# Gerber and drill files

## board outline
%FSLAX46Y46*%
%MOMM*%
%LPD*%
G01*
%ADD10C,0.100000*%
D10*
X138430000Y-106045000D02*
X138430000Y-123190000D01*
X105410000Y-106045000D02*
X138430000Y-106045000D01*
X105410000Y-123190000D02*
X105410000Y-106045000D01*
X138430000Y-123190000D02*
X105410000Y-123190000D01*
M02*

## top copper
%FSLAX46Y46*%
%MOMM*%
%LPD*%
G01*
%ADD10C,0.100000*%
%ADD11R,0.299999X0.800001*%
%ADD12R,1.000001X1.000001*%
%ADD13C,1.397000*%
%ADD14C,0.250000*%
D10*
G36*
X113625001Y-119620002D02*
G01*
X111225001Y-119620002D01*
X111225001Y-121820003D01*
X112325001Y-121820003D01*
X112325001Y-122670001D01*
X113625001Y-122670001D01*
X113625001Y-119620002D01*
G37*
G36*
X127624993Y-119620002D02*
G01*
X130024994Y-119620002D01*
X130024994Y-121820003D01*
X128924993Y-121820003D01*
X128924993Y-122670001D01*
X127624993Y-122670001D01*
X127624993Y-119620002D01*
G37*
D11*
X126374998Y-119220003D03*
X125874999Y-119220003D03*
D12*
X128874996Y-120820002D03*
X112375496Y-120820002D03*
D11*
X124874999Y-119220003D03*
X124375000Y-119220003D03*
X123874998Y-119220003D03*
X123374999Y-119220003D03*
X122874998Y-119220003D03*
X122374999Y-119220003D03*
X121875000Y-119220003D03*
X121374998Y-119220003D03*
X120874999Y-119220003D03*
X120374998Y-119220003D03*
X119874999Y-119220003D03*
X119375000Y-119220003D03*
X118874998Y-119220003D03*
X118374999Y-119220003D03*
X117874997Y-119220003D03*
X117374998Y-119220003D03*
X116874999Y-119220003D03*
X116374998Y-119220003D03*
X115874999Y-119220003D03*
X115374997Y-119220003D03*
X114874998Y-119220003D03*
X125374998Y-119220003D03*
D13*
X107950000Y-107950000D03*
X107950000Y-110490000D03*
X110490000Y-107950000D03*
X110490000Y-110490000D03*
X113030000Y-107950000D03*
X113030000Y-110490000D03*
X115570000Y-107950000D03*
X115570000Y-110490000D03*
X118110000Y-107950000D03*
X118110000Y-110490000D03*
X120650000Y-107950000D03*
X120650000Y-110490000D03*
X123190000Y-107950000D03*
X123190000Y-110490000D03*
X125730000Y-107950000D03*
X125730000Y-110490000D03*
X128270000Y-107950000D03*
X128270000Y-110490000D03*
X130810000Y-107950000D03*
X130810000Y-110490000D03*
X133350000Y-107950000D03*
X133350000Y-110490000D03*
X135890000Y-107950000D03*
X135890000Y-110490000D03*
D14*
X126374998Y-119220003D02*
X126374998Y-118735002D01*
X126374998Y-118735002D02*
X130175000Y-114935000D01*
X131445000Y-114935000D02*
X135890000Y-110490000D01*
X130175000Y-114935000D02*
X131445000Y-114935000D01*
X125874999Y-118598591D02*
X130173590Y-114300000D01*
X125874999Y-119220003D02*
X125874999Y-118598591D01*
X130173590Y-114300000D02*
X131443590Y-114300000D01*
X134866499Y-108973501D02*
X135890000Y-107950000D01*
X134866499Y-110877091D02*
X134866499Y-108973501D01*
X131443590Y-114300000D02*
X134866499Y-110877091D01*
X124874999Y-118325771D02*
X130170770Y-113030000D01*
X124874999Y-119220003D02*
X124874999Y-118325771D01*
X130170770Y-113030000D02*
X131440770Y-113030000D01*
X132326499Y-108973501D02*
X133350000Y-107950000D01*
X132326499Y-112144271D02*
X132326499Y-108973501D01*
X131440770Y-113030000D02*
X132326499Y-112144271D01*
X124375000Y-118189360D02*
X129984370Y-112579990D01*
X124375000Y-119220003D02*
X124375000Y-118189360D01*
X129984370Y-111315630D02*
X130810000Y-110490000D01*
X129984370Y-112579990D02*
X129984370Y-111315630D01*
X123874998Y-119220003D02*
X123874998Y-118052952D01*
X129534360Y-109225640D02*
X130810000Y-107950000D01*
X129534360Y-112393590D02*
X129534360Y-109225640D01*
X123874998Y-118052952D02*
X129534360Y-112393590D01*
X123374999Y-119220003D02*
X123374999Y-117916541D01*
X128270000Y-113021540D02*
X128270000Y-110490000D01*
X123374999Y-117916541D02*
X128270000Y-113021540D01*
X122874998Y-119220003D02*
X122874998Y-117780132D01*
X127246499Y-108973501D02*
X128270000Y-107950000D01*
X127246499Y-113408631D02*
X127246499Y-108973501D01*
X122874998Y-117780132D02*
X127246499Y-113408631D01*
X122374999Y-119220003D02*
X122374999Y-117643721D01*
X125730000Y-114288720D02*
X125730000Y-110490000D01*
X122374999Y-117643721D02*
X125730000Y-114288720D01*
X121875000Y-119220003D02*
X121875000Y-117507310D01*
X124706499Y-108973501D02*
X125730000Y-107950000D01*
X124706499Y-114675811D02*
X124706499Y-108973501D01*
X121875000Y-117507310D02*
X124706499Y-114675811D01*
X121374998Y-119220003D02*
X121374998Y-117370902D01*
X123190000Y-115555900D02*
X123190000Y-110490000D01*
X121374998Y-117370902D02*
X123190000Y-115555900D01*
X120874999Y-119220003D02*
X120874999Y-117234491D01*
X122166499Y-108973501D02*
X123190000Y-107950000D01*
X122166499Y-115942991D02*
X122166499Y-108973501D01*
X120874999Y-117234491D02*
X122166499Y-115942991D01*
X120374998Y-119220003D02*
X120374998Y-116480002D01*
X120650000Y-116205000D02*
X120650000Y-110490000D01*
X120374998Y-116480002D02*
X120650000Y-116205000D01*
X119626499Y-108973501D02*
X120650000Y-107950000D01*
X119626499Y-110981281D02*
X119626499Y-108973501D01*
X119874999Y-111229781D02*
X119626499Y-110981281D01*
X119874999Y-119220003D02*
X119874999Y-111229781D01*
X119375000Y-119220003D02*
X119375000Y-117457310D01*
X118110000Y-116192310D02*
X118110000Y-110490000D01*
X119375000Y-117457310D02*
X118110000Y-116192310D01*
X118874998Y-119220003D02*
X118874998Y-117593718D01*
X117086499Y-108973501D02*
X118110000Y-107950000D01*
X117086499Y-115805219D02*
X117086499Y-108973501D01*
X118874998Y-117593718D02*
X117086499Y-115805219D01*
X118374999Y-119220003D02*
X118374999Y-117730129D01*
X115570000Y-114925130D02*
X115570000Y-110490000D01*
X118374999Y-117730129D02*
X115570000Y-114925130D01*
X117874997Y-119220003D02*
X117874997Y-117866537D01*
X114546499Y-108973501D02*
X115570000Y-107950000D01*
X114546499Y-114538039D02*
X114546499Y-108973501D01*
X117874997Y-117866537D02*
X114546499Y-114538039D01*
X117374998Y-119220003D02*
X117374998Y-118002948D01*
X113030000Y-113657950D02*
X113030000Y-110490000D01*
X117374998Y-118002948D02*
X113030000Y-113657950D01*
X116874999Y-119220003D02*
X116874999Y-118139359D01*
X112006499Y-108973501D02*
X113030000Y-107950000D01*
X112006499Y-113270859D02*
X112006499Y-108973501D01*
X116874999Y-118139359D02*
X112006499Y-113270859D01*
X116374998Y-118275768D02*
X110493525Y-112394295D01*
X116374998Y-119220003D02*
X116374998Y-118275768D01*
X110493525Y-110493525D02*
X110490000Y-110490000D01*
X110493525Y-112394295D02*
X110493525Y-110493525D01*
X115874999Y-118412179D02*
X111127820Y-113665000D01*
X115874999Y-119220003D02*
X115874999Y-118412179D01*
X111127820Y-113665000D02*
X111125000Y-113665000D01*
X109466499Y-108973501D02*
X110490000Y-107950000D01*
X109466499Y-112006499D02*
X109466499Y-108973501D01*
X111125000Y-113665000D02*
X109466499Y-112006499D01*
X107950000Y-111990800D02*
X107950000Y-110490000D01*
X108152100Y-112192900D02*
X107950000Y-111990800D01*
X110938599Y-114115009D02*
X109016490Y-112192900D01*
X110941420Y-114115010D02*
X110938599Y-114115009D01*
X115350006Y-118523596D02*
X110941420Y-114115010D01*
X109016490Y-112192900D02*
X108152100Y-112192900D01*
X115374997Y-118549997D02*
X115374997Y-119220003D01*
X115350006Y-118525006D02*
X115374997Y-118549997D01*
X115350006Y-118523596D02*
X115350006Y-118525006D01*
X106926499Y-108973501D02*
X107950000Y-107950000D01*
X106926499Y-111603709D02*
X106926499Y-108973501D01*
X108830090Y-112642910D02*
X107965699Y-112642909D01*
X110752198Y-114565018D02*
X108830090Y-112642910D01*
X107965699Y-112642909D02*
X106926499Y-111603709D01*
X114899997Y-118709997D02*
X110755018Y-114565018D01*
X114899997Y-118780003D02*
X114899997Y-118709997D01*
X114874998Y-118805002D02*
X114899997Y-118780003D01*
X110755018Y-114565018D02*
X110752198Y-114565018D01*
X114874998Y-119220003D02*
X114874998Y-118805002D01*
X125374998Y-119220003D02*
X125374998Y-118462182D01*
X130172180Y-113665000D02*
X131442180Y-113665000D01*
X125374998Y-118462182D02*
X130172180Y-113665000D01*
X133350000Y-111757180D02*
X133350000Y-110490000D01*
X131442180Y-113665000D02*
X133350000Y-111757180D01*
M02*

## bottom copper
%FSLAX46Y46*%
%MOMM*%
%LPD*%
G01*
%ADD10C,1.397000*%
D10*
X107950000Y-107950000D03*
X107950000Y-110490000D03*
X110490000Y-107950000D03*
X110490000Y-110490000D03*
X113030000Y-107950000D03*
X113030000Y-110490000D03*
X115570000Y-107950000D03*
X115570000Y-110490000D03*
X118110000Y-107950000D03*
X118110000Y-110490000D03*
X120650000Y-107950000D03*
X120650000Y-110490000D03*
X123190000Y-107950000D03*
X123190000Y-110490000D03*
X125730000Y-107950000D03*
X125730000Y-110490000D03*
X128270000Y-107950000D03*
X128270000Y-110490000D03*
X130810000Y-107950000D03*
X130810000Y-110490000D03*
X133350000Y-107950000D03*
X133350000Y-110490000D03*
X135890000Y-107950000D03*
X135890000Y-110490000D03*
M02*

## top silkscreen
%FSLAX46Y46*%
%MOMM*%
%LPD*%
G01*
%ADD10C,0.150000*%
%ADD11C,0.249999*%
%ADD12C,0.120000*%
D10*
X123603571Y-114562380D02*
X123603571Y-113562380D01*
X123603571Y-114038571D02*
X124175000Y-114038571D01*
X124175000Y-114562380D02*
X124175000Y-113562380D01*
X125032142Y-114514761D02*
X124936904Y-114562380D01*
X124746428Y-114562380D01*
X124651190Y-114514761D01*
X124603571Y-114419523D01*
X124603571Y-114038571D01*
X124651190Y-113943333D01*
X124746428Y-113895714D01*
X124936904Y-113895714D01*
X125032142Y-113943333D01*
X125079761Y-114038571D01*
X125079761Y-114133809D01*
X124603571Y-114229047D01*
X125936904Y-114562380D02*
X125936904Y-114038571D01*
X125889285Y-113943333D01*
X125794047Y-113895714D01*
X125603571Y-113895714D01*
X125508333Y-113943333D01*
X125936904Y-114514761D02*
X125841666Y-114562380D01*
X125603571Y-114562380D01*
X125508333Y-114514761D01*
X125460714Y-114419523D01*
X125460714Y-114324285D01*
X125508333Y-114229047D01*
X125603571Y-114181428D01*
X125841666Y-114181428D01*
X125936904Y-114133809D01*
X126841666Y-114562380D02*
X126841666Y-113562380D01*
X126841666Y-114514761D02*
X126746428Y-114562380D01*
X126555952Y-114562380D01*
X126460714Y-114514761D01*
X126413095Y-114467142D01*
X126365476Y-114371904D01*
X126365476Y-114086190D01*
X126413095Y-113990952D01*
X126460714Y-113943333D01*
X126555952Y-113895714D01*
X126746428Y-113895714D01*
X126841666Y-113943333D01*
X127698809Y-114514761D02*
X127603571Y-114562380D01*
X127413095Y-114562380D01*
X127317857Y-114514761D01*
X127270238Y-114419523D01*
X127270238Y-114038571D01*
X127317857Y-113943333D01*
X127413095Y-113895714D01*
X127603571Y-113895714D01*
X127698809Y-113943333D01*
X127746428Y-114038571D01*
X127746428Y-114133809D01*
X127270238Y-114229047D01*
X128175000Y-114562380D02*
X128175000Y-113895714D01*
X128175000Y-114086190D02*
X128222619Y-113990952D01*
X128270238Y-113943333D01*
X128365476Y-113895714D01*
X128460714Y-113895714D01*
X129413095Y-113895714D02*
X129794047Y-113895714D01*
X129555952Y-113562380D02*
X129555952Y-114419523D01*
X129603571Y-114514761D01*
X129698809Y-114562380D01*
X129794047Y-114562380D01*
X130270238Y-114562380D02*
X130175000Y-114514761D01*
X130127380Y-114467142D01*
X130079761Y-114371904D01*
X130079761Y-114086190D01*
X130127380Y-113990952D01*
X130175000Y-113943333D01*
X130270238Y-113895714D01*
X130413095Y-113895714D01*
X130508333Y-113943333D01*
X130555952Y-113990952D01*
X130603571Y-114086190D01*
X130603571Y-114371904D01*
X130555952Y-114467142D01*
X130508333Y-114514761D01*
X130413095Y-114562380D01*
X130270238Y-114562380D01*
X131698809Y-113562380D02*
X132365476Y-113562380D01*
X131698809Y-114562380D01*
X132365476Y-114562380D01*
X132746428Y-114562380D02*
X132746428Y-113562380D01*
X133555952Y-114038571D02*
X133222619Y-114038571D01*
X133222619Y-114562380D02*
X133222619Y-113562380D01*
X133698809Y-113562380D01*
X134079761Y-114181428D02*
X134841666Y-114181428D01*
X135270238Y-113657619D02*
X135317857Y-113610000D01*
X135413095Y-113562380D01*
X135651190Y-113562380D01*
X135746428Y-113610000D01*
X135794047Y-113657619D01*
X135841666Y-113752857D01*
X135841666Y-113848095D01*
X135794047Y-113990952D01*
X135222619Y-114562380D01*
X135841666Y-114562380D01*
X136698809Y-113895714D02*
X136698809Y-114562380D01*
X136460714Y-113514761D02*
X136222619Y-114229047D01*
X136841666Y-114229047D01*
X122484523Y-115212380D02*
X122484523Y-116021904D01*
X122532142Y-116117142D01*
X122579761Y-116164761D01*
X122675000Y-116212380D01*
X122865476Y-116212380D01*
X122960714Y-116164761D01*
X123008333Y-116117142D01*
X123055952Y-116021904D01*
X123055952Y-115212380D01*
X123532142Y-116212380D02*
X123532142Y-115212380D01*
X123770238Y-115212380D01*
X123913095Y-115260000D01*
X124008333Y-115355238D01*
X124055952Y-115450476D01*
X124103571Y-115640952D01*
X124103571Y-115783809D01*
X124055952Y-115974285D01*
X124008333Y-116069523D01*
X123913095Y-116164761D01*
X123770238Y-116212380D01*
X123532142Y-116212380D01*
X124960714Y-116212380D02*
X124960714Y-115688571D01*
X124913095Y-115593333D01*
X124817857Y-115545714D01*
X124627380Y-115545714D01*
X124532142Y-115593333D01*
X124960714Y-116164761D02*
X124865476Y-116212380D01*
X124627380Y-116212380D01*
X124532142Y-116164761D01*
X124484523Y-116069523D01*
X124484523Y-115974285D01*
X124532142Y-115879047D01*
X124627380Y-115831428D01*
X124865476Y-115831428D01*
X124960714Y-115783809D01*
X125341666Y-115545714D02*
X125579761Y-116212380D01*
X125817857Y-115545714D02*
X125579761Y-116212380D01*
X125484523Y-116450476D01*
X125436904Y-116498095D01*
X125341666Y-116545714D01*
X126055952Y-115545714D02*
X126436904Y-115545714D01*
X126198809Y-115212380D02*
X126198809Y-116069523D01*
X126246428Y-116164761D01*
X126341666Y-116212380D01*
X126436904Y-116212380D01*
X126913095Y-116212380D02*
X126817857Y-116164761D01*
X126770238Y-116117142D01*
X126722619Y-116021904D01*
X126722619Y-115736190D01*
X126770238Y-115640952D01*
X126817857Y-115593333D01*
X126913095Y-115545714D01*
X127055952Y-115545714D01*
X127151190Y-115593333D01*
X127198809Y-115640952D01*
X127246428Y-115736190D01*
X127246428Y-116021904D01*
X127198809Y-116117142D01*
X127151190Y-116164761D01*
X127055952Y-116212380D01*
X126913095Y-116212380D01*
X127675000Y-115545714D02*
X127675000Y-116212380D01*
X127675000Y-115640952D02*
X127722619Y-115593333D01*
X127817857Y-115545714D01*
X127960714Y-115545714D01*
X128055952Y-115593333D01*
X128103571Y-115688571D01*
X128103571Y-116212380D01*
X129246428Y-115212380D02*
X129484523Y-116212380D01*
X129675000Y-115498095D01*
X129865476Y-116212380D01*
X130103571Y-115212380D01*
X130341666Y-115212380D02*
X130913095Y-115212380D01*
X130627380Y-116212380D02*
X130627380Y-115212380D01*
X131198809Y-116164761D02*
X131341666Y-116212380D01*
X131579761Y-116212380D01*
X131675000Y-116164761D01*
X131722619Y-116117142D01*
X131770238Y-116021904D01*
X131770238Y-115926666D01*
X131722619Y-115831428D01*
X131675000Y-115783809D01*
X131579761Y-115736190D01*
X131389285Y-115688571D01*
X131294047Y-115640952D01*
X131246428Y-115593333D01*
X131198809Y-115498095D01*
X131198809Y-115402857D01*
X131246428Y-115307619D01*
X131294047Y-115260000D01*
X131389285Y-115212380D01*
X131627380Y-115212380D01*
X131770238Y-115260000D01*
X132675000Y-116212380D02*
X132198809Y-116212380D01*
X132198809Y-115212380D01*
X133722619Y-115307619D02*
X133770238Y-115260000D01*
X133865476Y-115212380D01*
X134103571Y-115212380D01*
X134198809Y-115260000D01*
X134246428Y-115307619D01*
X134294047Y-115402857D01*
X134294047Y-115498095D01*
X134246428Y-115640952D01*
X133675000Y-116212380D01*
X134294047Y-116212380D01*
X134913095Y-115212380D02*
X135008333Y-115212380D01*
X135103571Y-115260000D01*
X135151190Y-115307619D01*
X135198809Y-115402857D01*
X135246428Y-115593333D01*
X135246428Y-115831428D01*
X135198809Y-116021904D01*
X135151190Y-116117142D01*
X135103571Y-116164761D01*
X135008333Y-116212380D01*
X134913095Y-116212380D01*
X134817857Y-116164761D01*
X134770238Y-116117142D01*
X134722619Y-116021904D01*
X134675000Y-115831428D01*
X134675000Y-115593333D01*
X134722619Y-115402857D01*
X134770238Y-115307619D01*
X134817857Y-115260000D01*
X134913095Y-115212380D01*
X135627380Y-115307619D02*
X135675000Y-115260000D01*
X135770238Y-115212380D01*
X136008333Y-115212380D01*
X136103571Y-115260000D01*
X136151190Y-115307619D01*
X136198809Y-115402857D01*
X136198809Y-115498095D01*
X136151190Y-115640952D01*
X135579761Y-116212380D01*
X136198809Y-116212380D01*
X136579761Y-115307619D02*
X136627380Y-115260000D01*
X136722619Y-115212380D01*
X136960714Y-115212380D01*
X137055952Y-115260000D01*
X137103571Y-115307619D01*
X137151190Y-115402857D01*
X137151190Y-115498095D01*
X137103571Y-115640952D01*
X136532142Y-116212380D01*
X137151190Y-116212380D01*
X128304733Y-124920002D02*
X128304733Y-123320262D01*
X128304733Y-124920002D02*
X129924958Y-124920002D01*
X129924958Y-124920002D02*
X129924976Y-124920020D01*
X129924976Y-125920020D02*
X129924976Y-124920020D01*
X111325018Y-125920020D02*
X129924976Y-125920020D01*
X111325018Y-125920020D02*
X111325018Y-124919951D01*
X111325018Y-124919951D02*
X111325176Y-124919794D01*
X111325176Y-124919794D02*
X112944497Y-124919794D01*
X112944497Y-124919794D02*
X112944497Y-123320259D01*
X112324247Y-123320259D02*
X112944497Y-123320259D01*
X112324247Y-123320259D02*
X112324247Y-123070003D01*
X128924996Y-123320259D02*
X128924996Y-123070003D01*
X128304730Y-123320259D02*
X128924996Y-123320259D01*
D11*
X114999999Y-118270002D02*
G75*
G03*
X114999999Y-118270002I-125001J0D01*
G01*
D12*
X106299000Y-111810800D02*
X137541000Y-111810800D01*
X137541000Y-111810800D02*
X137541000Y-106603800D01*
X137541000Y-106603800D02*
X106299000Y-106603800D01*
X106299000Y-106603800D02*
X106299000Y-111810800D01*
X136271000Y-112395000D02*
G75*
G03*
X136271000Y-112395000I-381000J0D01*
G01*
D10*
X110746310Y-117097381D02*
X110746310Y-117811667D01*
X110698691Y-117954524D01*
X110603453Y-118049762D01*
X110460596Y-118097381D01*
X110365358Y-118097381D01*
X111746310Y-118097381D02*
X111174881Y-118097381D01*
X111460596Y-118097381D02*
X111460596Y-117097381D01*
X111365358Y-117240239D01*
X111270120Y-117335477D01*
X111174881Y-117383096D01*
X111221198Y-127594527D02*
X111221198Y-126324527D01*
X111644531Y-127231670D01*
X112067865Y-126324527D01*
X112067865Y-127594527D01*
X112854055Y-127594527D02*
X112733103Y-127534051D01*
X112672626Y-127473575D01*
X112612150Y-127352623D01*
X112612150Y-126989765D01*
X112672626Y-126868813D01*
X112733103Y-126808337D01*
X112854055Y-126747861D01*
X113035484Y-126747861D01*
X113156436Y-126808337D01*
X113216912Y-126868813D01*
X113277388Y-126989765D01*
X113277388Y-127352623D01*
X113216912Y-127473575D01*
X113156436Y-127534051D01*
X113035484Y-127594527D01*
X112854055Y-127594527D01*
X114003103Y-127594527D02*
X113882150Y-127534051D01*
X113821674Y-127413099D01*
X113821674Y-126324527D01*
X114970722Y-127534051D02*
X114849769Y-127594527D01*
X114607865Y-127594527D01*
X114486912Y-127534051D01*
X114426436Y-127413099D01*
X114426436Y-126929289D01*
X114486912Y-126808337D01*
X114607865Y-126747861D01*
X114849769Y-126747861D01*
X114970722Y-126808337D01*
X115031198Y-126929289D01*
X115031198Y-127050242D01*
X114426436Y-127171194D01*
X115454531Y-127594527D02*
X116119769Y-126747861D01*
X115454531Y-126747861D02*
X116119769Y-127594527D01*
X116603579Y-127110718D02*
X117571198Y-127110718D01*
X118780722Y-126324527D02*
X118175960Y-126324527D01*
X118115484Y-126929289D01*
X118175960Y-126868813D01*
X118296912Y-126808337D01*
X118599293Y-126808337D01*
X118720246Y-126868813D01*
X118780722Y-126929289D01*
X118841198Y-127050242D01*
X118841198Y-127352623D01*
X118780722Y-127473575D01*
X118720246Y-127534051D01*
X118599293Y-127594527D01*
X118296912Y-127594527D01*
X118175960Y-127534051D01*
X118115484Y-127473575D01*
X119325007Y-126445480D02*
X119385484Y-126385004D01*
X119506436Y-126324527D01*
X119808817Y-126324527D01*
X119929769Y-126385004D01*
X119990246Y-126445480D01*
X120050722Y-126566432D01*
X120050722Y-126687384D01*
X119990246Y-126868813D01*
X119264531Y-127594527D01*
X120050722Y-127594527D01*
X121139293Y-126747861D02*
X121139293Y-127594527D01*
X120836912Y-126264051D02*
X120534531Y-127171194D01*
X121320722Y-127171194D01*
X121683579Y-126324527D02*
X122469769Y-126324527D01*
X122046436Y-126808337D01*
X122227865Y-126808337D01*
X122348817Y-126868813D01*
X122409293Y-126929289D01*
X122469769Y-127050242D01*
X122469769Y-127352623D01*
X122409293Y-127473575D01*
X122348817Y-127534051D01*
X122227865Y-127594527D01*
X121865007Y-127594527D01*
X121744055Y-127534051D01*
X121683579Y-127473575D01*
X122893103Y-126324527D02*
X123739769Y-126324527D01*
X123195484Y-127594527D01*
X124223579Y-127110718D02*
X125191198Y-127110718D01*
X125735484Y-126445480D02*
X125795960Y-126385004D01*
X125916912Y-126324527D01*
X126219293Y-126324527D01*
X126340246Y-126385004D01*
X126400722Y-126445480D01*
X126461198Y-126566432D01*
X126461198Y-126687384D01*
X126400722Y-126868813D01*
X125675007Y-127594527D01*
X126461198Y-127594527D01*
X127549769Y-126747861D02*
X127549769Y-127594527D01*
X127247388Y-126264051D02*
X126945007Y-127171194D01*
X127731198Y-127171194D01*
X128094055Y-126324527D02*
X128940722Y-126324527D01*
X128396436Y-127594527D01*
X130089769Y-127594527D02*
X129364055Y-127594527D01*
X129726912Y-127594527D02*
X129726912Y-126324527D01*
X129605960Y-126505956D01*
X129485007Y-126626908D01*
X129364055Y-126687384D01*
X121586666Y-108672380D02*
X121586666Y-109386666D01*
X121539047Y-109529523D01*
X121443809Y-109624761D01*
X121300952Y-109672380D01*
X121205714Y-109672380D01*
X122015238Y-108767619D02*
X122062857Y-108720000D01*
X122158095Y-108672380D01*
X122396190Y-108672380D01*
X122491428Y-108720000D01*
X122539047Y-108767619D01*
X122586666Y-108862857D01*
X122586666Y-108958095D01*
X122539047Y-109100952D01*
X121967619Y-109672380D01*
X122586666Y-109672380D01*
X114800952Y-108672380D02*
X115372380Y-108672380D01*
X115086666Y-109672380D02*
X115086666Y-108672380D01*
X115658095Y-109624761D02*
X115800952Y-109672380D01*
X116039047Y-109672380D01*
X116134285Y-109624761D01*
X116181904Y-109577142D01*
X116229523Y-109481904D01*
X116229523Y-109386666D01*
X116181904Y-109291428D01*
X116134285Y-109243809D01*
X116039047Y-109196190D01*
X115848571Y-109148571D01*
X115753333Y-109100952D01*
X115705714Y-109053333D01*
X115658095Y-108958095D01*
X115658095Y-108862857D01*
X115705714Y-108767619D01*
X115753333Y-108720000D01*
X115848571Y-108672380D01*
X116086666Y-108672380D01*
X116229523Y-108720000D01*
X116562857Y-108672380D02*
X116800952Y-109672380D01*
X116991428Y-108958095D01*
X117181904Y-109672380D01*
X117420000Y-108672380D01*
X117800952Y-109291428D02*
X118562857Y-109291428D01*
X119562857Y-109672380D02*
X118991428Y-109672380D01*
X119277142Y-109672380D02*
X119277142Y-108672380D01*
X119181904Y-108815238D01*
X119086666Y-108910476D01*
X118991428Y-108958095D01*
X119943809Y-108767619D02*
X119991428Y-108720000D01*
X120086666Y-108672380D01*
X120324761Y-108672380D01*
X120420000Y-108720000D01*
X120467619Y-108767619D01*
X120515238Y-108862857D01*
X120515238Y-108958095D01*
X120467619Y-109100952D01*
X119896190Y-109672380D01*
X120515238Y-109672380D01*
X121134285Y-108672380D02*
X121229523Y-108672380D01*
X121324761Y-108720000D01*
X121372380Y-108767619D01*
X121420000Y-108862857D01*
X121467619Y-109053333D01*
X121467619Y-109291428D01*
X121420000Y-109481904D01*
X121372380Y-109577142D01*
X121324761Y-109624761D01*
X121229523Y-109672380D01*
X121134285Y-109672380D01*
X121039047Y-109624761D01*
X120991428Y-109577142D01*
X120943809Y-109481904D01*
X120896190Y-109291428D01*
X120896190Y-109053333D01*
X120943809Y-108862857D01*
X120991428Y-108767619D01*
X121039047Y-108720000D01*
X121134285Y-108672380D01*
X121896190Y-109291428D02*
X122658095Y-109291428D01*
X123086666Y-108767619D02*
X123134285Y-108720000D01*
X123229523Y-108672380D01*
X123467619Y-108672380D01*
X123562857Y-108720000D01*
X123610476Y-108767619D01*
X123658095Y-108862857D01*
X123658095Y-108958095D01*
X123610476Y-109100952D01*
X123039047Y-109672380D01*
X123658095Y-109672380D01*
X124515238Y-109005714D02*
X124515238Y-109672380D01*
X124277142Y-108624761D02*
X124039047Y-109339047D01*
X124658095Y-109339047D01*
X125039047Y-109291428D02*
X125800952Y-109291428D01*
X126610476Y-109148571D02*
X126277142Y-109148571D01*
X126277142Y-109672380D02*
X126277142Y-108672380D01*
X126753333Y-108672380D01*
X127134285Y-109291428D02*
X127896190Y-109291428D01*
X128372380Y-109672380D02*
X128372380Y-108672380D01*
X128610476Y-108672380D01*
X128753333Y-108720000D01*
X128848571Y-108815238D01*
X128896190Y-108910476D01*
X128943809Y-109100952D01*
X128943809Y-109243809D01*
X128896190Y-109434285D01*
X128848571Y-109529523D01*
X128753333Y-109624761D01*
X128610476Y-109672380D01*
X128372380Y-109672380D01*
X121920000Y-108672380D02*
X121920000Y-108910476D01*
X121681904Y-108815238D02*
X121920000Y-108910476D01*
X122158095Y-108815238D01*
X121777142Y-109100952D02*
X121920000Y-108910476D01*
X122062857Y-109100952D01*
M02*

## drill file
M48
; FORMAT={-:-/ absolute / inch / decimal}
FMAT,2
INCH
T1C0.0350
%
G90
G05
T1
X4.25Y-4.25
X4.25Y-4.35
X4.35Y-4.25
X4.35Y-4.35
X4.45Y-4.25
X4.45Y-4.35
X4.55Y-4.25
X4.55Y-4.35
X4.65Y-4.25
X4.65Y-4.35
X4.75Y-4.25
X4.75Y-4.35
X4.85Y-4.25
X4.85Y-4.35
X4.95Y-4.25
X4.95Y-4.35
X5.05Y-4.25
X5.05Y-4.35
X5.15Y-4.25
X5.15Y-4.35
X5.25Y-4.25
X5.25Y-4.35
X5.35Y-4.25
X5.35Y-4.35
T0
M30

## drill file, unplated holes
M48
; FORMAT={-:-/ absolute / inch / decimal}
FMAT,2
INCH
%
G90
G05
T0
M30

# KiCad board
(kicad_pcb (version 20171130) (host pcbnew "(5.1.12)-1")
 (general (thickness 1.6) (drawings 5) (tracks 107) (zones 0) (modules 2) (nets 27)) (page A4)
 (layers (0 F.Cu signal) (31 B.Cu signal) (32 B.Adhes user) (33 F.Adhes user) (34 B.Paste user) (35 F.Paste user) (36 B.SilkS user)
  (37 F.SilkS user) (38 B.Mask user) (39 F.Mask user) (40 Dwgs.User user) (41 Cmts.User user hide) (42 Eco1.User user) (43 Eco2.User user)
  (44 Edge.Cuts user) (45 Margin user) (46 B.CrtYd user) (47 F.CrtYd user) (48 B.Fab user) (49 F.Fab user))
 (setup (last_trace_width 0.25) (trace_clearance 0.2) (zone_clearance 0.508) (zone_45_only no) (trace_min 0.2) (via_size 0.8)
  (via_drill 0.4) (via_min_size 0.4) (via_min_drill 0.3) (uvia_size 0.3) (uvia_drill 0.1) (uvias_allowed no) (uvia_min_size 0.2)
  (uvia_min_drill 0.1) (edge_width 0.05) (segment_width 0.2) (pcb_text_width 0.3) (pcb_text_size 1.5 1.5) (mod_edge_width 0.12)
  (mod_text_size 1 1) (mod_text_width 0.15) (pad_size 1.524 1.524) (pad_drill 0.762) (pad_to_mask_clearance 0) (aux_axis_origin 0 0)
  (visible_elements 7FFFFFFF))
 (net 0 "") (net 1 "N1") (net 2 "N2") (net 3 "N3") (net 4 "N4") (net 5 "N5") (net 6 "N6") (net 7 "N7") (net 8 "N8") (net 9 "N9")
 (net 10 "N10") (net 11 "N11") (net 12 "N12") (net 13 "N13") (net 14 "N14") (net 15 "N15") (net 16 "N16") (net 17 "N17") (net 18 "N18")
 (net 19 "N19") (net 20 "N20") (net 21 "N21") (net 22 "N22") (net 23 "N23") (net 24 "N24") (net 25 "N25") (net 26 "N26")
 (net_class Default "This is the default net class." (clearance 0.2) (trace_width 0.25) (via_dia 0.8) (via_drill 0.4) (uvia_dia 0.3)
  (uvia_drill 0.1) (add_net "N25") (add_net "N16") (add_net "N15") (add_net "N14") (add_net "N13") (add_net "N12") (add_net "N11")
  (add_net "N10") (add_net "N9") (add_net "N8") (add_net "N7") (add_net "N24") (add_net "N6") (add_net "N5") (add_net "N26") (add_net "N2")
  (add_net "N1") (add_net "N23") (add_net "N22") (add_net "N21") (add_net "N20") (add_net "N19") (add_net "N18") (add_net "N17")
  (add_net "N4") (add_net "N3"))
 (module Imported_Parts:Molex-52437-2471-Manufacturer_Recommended (layer F.Cu) (at 120.625246 120.020004)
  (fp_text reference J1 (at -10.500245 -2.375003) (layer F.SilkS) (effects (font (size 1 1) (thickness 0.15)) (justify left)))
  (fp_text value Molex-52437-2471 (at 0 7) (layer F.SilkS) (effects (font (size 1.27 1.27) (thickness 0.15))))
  (fp_poly
   (pts (xy -7.000245 -0.400002) (xy -9.400245 -0.400002) (xy -9.400245 1.799999) (xy -8.300245 1.799999) (xy -8.300245 2.649997)
    (xy -7.000245 2.649997))
   (layer F.Cu) (width 0))
  (fp_poly
   (pts (xy 6.999747 -0.400002) (xy 9.399748 -0.400002) (xy 9.399748 1.799999) (xy 8.299747 1.799999) (xy 8.299747 2.649997)
    (xy 6.999747 2.649997))
   (layer F.Cu) (width 0))
  (fp_line (start 7.679487 4.899998) (end 7.679487 3.300258) (layer F.SilkS) (width 0.15))
  (fp_line (start 7.679487 4.899998) (end 9.299712 4.899998) (layer F.SilkS) (width 0.15))
  (fp_line (start 9.299712 4.899998) (end 9.29973 4.900016) (layer F.SilkS) (width 0.15))
  (fp_line (start 9.29973 5.900016) (end 9.29973 4.900016) (layer F.SilkS) (width 0.15))
  (fp_line (start -9.300228 5.900016) (end 9.29973 5.900016) (layer F.SilkS) (width 0.15))
  (fp_line (start -9.300228 5.900016) (end -9.300228 4.899947) (layer F.SilkS) (width 0.15))
  (fp_line (start -9.300228 4.899947) (end -9.30007 4.89979) (layer F.SilkS) (width 0.15))
  (fp_line (start -9.30007 4.89979) (end -7.680749 4.89979) (layer F.SilkS) (width 0.15))
  (fp_line (start -7.680749 4.89979) (end -7.680749 3.300255) (layer F.SilkS) (width 0.15))
  (fp_line (start -8.300999 3.300255) (end -7.680749 3.300255) (layer F.SilkS) (width 0.15))
  (fp_line (start -8.300999 3.300255) (end -8.300999 3.049999) (layer F.SilkS) (width 0.15))
  (fp_line (start 8.29975 3.300255) (end 8.29975 3.049999) (layer F.SilkS) (width 0.15))
  (fp_line (start 7.679484 3.300255) (end 8.29975 3.300255) (layer F.SilkS) (width 0.15))
  (fp_circle (center -5.750248 -1.750002) (end -5.625247 -1.750002) (layer F.SilkS) (width 0.249999))
  (pad 24 smd rect (at 5.749752 -0.800001) (size 0.299999 0.800001) (layers F.Cu F.Paste F.Mask) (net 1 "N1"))
  (pad 23 smd rect (at 5.249753 -0.800001) (size 0.299999 0.800001) (layers F.Cu F.Paste F.Mask) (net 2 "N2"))
  (pad MP2 smd rect (at 8.24975 0.799998 180) (size 1.000001 1.000001) (layers F.Cu F.Paste F.Mask) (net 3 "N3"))
  (pad MP1 smd rect (at -8.24975 0.799998 180) (size 1.000001 1.000001) (layers F.Cu F.Paste F.Mask) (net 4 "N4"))
  (pad 21 smd rect (at 4.249753 -0.800001 180) (size 0.299999 0.800001) (layers F.Cu F.Paste F.Mask) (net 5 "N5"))
  (pad 20 smd rect (at 3.749754 -0.800001 180) (size 0.299999 0.800001) (layers F.Cu F.Paste F.Mask) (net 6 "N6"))
  (pad 19 smd rect (at 3.249752 -0.800001 180) (size 0.299999 0.800001) (layers F.Cu F.Paste F.Mask) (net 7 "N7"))
  (pad 18 smd rect (at 2.749753 -0.800001 180) (size 0.299999 0.800001) (layers F.Cu F.Paste F.Mask) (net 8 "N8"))
  (pad 17 smd rect (at 2.249752 -0.800001 180) (size 0.299999 0.800001) (layers F.Cu F.Paste F.Mask) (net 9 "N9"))
  (pad 16 smd rect (at 1.749753 -0.800001 180) (size 0.299999 0.800001) (layers F.Cu F.Paste F.Mask) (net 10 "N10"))
  (pad 15 smd rect (at 1.249754 -0.800001 180) (size 0.299999 0.800001) (layers F.Cu F.Paste F.Mask) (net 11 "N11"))
  (pad 14 smd rect (at 0.749752 -0.800001 180) (size 0.299999 0.800001) (layers F.Cu F.Paste F.Mask) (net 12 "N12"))
  (pad 13 smd rect (at 0.249753 -0.800001 180) (size 0.299999 0.800001) (layers F.Cu F.Paste F.Mask) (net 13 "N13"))
  (pad 12 smd rect (at -0.250248 -0.800001 180) (size 0.299999 0.800001) (layers F.Cu F.Paste F.Mask) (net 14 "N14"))
  (pad 11 smd rect (at -0.750247 -0.800001 180) (size 0.299999 0.800001) (layers F.Cu F.Paste F.Mask) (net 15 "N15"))
  (pad 10 smd rect (at -1.250246 -0.800001 180) (size 0.299999 0.800001) (layers F.Cu F.Paste F.Mask) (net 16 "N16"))
  (pad 9 smd rect (at -1.750248 -0.800001 180) (size 0.299999 0.800001) (layers F.Cu F.Paste F.Mask) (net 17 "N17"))
  (pad 8 smd rect (at -2.250247 -0.800001 180) (size 0.299999 0.800001) (layers F.Cu F.Paste F.Mask) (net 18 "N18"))
  (pad 7 smd rect (at -2.750249 -0.800001 180) (size 0.299999 0.800001) (layers F.Cu F.Paste F.Mask) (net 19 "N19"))
  (pad 6 smd rect (at -3.250248 -0.800001 180) (size 0.299999 0.800001) (layers F.Cu F.Paste F.Mask) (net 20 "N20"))
  (pad 5 smd rect (at -3.750247 -0.800001 180) (size 0.299999 0.800001) (layers F.Cu F.Paste F.Mask) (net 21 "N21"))
  (pad 4 smd rect (at -4.250248 -0.800001 180) (size 0.299999 0.800001) (layers F.Cu F.Paste F.Mask) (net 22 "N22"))
  (pad 3 smd rect (at -4.750247 -0.800001 180) (size 0.299999 0.800001) (layers F.Cu F.Paste F.Mask) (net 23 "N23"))
  (pad 2 smd rect (at -5.250249 -0.800001 180) (size 0.299999 0.800001) (layers F.Cu F.Paste F.Mask) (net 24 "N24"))
  (pad 1 smd rect (at -5.750248 -0.800001 180) (size 0.299999 0.800001) (layers F.Cu F.Paste F.Mask) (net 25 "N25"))
  (pad 22 smd rect (at 4.749752 -0.800001) (size 0.299999 0.800001) (layers F.Cu F.Paste F.Mask) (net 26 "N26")))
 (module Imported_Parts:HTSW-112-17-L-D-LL (layer F.Cu) (at 121.92 109.22)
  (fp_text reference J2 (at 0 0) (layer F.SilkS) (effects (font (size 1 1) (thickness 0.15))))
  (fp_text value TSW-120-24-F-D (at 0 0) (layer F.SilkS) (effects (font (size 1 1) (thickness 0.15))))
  (fp_line (start -15.621 2.5908) (end 15.621 2.5908) (layer F.SilkS) (width 0.12))
  (fp_line (start 15.621 2.5908) (end 15.621 -2.6162) (layer F.SilkS) (width 0.12))
  (fp_line (start 15.621 -2.6162) (end -15.621 -2.6162) (layer F.SilkS) (width 0.12))
  (fp_line (start -15.621 -2.6162) (end -15.621 2.5908) (layer F.SilkS) (width 0.12))
  (fp_circle (center 13.97 3.175) (end 14.351 3.175) (layer F.SilkS) (width 0.12))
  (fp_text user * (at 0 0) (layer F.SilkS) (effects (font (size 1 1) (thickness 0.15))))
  (pad 24 thru_hole circle (at -13.97 -1.27 90) (size 1.397 1.397) (drill 0.889) (layers *.Cu *.Mask) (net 25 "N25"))
  (pad 23 thru_hole circle (at -13.97 1.27 90) (size 1.397 1.397) (drill 0.889) (layers *.Cu *.Mask) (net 24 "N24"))
  (pad 22 thru_hole circle (at -11.43 -1.27 90) (size 1.397 1.397) (drill 0.889) (layers *.Cu *.Mask) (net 23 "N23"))
  (pad 21 thru_hole circle (at -11.43 1.27 90) (size 1.397 1.397) (drill 0.889) (layers *.Cu *.Mask) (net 22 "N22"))
  (pad 20 thru_hole circle (at -8.89 -1.27 90) (size 1.397 1.397) (drill 0.889) (layers *.Cu *.Mask) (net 21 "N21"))
  (pad 19 thru_hole circle (at -8.89 1.27 90) (size 1.397 1.397) (drill 0.889) (layers *.Cu *.Mask) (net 20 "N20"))
  (pad 18 thru_hole circle (at -6.35 -1.27 90) (size 1.397 1.397) (drill 0.889) (layers *.Cu *.Mask) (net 19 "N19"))
  (pad 17 thru_hole circle (at -6.35 1.27 90) (size 1.397 1.397) (drill 0.889) (layers *.Cu *.Mask) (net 18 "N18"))
  (pad 16 thru_hole circle (at -3.81 -1.27 90) (size 1.397 1.397) (drill 0.889) (layers *.Cu *.Mask) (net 17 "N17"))
  (pad 15 thru_hole circle (at -3.81 1.27 90) (size 1.397 1.397) (drill 0.889) (layers *.Cu *.Mask) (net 16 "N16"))
  (pad 14 thru_hole circle (at -1.27 -1.27 90) (size 1.397 1.397) (drill 0.889) (layers *.Cu *.Mask) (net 15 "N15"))
  (pad 13 thru_hole circle (at -1.27 1.27 90) (size 1.397 1.397) (drill 0.889) (layers *.Cu *.Mask) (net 14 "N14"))
  (pad 12 thru_hole circle (at 1.27 -1.27 90) (size 1.397 1.397) (drill 0.889) (layers *.Cu *.Mask) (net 13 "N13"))
  (pad 11 thru_hole circle (at 1.27 1.27 90) (size 1.397 1.397) (drill 0.889) (layers *.Cu *.Mask) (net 12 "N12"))
  (pad 10 thru_hole circle (at 3.81 -1.27 90) (size 1.397 1.397) (drill 0.889) (layers *.Cu *.Mask) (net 11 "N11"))
  (pad 9 thru_hole circle (at 3.81 1.27 90) (size 1.397 1.397) (drill 0.889) (layers *.Cu *.Mask) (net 10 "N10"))
  (pad 8 thru_hole circle (at 6.35 -1.27 90) (size 1.397 1.397) (drill 0.889) (layers *.Cu *.Mask) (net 9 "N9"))
  (pad 7 thru_hole circle (at 6.35 1.27 90) (size 1.397 1.397) (drill 0.889) (layers *.Cu *.Mask) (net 8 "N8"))
  (pad 6 thru_hole circle (at 8.89 -1.27 90) (size 1.397 1.397) (drill 0.889) (layers *.Cu *.Mask) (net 7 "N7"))
  (pad 5 thru_hole circle (at 8.89 1.27 90) (size 1.397 1.397) (drill 0.889) (layers *.Cu *.Mask) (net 6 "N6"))
  (pad 4 thru_hole circle (at 11.43 -1.27 90) (size 1.397 1.397) (drill 0.889) (layers *.Cu *.Mask) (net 5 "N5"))
  (pad 3 thru_hole circle (at 11.43 1.27 90) (size 1.397 1.397) (drill 0.889) (layers *.Cu *.Mask) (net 26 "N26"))
  (pad 2 thru_hole circle (at 13.97 -1.27 90) (size 1.397 1.397) (drill 0.889) (layers *.Cu *.Mask) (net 2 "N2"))
  (pad 1 thru_hole circle (at 13.97 1.27 90) (size 1.397 1.397) (drill 0.889) (layers *.Cu *.Mask) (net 1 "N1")))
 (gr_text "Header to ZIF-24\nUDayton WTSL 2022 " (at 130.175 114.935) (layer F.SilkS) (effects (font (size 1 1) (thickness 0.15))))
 (gr_line (start 138.43 106.045) (end 138.43 123.19) (layer Edge.Cuts) (width 0.1))
 (gr_line (start 105.41 106.045) (end 138.43 106.045) (layer Edge.Cuts) (width 0.1))
 (gr_line (start 105.41 123.19) (end 105.41 106.045) (layer Edge.Cuts) (width 0.1))
 (gr_line (start 138.43 123.19) (end 105.41 123.19) (layer Edge.Cuts) (width 0.1))
 (segment (start 126.374998 119.220003) (end 126.374998 118.735002) (width 0.25) (layer F.Cu) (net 1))
 (segment (start 126.374998 118.735002) (end 130.175 114.935) (width 0.25) (layer F.Cu) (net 1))
 (segment (start 131.445 114.935) (end 135.89 110.49) (width 0.25) (layer F.Cu) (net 1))
 (segment (start 130.175 114.935) (end 131.445 114.935) (width 0.25) (layer F.Cu) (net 1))
 (segment (start 125.874999 118.598591) (end 130.17359 114.3) (width 0.25) (layer F.Cu) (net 2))
 (segment (start 125.874999 119.220003) (end 125.874999 118.598591) (width 0.25) (layer F.Cu) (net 2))
 (segment (start 130.17359 114.3) (end 131.44359 114.3) (width 0.25) (layer F.Cu) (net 2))
 (segment (start 134.866499 108.973501) (end 135.89 107.95) (width 0.25) (layer F.Cu) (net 2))
 (segment (start 134.866499 110.877091) (end 134.866499 108.973501) (width 0.25) (layer F.Cu) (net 2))
 (segment (start 131.44359 114.3) (end 134.866499 110.877091) (width 0.25) (layer F.Cu) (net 2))
 (segment (start 124.874999 118.325771) (end 130.17077 113.03) (width 0.25) (layer F.Cu) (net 5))
 (segment (start 124.874999 119.220003) (end 124.874999 118.325771) (width 0.25) (layer F.Cu) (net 5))
 (segment (start 130.17077 113.03) (end 131.44077 113.03) (width 0.25) (layer F.Cu) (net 5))
 (segment (start 132.326499 108.973501) (end 133.35 107.95) (width 0.25) (layer F.Cu) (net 5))
 (segment (start 132.326499 112.144271) (end 132.326499 108.973501) (width 0.25) (layer F.Cu) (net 5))
 (segment (start 131.44077 113.03) (end 132.326499 112.144271) (width 0.25) (layer F.Cu) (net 5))
 (segment (start 124.375 118.18936) (end 129.98437 112.57999) (width 0.25) (layer F.Cu) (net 6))
 (segment (start 124.375 119.220003) (end 124.375 118.18936) (width 0.25) (layer F.Cu) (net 6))
 (segment (start 129.98437 111.31563) (end 130.81 110.49) (width 0.25) (layer F.Cu) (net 6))
 (segment (start 129.98437 112.57999) (end 129.98437 111.31563) (width 0.25) (layer F.Cu) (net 6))
 (segment (start 123.874998 119.220003) (end 123.874998 118.052952) (width 0.25) (layer F.Cu) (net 7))
 (segment (start 129.53436 109.22564) (end 130.81 107.95) (width 0.25) (layer F.Cu) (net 7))
 (segment (start 129.53436 112.39359) (end 129.53436 109.22564) (width 0.25) (layer F.Cu) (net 7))
 (segment (start 123.874998 118.052952) (end 129.53436 112.39359) (width 0.25) (layer F.Cu) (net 7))
 (segment (start 123.374999 119.220003) (end 123.374999 117.916541) (width 0.25) (layer F.Cu) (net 8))
 (segment (start 128.27 113.02154) (end 128.27 110.49) (width 0.25) (layer F.Cu) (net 8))
 (segment (start 123.374999 117.916541) (end 128.27 113.02154) (width 0.25) (layer F.Cu) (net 8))
 (segment (start 122.874998 119.220003) (end 122.874998 117.780132) (width 0.25) (layer F.Cu) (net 9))
 (segment (start 127.246499 108.973501) (end 128.27 107.95) (width 0.25) (layer F.Cu) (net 9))
 (segment (start 127.246499 113.408631) (end 127.246499 108.973501) (width 0.25) (layer F.Cu) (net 9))
 (segment (start 122.874998 117.780132) (end 127.246499 113.408631) (width 0.25) (layer F.Cu) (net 9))
 (segment (start 122.374999 119.220003) (end 122.374999 117.643721) (width 0.25) (layer F.Cu) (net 10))
 (segment (start 125.73 114.28872) (end 125.73 110.49) (width 0.25) (layer F.Cu) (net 10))
 (segment (start 122.374999 117.643721) (end 125.73 114.28872) (width 0.25) (layer F.Cu) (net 10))
 (segment (start 121.875 119.220003) (end 121.875 117.50731) (width 0.25) (layer F.Cu) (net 11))
 (segment (start 124.706499 108.973501) (end 125.73 107.95) (width 0.25) (layer F.Cu) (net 11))
 (segment (start 124.706499 114.675811) (end 124.706499 108.973501) (width 0.25) (layer F.Cu) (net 11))
 (segment (start 121.875 117.50731) (end 124.706499 114.675811) (width 0.25) (layer F.Cu) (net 11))
 (segment (start 121.374998 119.220003) (end 121.374998 117.370902) (width 0.25) (layer F.Cu) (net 12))
 (segment (start 123.19 115.5559) (end 123.19 110.49) (width 0.25) (layer F.Cu) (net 12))
 (segment (start 121.374998 117.370902) (end 123.19 115.5559) (width 0.25) (layer F.Cu) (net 12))
 (segment (start 120.874999 119.220003) (end 120.874999 117.234491) (width 0.25) (layer F.Cu) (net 13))
 (segment (start 122.166499 108.973501) (end 123.19 107.95) (width 0.25) (layer F.Cu) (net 13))
 (segment (start 122.166499 115.942991) (end 122.166499 108.973501) (width 0.25) (layer F.Cu) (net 13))
 (segment (start 120.874999 117.234491) (end 122.166499 115.942991) (width 0.25) (layer F.Cu) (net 13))
 (segment (start 120.374998 119.220003) (end 120.374998 116.480002) (width 0.25) (layer F.Cu) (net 14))
 (segment (start 120.65 116.205) (end 120.65 110.49) (width 0.25) (layer F.Cu) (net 14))
 (segment (start 120.374998 116.480002) (end 120.65 116.205) (width 0.25) (layer F.Cu) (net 14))
 (segment (start 119.626499 108.973501) (end 120.65 107.95) (width 0.25) (layer F.Cu) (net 15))
 (segment (start 119.626499 110.981281) (end 119.626499 108.973501) (width 0.25) (layer F.Cu) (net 15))
 (segment (start 119.874999 111.229781) (end 119.626499 110.981281) (width 0.25) (layer F.Cu) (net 15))
 (segment (start 119.874999 119.220003) (end 119.874999 111.229781) (width 0.25) (layer F.Cu) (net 15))
 (segment (start 119.375 119.220003) (end 119.375 117.45731) (width 0.25) (layer F.Cu) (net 16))
 (segment (start 118.11 116.19231) (end 118.11 110.49) (width 0.25) (layer F.Cu) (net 16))
 (segment (start 119.375 117.45731) (end 118.11 116.19231) (width 0.25) (layer F.Cu) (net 16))
 (segment (start 118.874998 119.220003) (end 118.874998 117.593718) (width 0.25) (layer F.Cu) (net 17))
 (segment (start 117.086499 108.973501) (end 118.11 107.95) (width 0.25) (layer F.Cu) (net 17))
 (segment (start 117.086499 115.805219) (end 117.086499 108.973501) (width 0.25) (layer F.Cu) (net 17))
 (segment (start 118.874998 117.593718) (end 117.086499 115.805219) (width 0.25) (layer F.Cu) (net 17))
 (segment (start 118.374999 119.220003) (end 118.374999 117.730129) (width 0.25) (layer F.Cu) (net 18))
 (segment (start 115.57 114.92513) (end 115.57 110.49) (width 0.25) (layer F.Cu) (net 18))
 (segment (start 118.374999 117.730129) (end 115.57 114.92513) (width 0.25) (layer F.Cu) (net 18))
 (segment (start 117.874997 119.220003) (end 117.874997 117.866537) (width 0.25) (layer F.Cu) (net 19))
 (segment (start 114.546499 108.973501) (end 115.57 107.95) (width 0.25) (layer F.Cu) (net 19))
 (segment (start 114.546499 114.538039) (end 114.546499 108.973501) (width 0.25) (layer F.Cu) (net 19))
 (segment (start 117.874997 117.866537) (end 114.546499 114.538039) (width 0.25) (layer F.Cu) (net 19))
 (segment (start 117.374998 119.220003) (end 117.374998 118.002948) (width 0.25) (layer F.Cu) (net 20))
 (segment (start 113.03 113.65795) (end 113.03 110.49) (width 0.25) (layer F.Cu) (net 20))
 (segment (start 117.374998 118.002948) (end 113.03 113.65795) (width 0.25) (layer F.Cu) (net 20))
 (segment (start 116.874999 119.220003) (end 116.874999 118.139359) (width 0.25) (layer F.Cu) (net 21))
 (segment (start 112.006499 108.973501) (end 113.03 107.95) (width 0.25) (layer F.Cu) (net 21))
 (segment (start 112.006499 113.270859) (end 112.006499 108.973501) (width 0.25) (layer F.Cu) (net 21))
 (segment (start 116.874999 118.139359) (end 112.006499 113.270859) (width 0.25) (layer F.Cu) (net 21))
 (segment (start 116.374998 118.275768) (end 110.493525 112.394295) (width 0.25) (layer F.Cu) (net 22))
 (segment (start 116.374998 119.220003) (end 116.374998 118.275768) (width 0.25) (layer F.Cu) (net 22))
 (segment (start 110.493525 110.493525) (end 110.49 110.49) (width 0.25) (layer F.Cu) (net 22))
 (segment (start 110.493525 112.394295) (end 110.493525 110.493525) (width 0.25) (layer F.Cu) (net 22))
 (segment (start 115.874999 118.412179) (end 111.12782 113.665) (width 0.25) (layer F.Cu) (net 23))
 (segment (start 115.874999 119.220003) (end 115.874999 118.412179) (width 0.25) (layer F.Cu) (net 23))
 (segment (start 111.12782 113.665) (end 111.125 113.665) (width 0.25) (layer F.Cu) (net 23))
 (segment (start 109.466499 108.973501) (end 110.49 107.95) (width 0.25) (layer F.Cu) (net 23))
 (segment (start 109.466499 112.006499) (end 109.466499 108.973501) (width 0.25) (layer F.Cu) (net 23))
 (segment (start 111.125 113.665) (end 109.466499 112.006499) (width 0.25) (layer F.Cu) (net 23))
 (segment (start 107.95 111.9908) (end 107.95 110.49) (width 0.25) (layer F.Cu) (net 24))
 (segment (start 108.1521 112.1929) (end 107.95 111.9908) (width 0.25) (layer F.Cu) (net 24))
 (segment (start 110.938599 114.115009) (end 109.01649 112.1929) (width 0.25) (layer F.Cu) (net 24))
 (segment (start 110.94142 114.11501) (end 110.938599 114.115009) (width 0.25) (layer F.Cu) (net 24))
 (segment (start 115.350006 118.523596) (end 110.94142 114.11501) (width 0.25) (layer F.Cu) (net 24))
 (segment (start 109.01649 112.1929) (end 108.1521 112.1929) (width 0.25) (layer F.Cu) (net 24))
 (segment (start 115.374997 118.549997) (end 115.374997 119.220003) (width 0.25) (layer F.Cu) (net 24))
 (segment (start 115.350006 118.525006) (end 115.374997 118.549997) (width 0.25) (layer F.Cu) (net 24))
 (segment (start 115.350006 118.523596) (end 115.350006 118.525006) (width 0.25) (layer F.Cu) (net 24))
 (segment (start 106.926499 108.973501) (end 107.95 107.95) (width 0.25) (layer F.Cu) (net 25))
 (segment (start 106.926499 111.603709) (end 106.926499 108.973501) (width 0.25) (layer F.Cu) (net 25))
 (segment (start 108.83009 112.64291) (end 107.965699 112.642909) (width 0.25) (layer F.Cu) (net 25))
 (segment (start 110.752198 114.565018) (end 108.83009 112.64291) (width 0.25) (layer F.Cu) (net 25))
 (segment (start 107.965699 112.642909) (end 106.926499 111.603709) (width 0.25) (layer F.Cu) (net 25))
 (segment (start 114.899997 118.709997) (end 110.755018 114.565018) (width 0.25) (layer F.Cu) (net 25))
 (segment (start 114.899997 118.780003) (end 114.899997 118.709997) (width 0.25) (layer F.Cu) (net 25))
 (segment (start 114.874998 118.805002) (end 114.899997 118.780003) (width 0.25) (layer F.Cu) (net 25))
 (segment (start 110.755018 114.565018) (end 110.752198 114.565018) (width 0.25) (layer F.Cu) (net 25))
 (segment (start 114.874998 119.220003) (end 114.874998 118.805002) (width 0.25) (layer F.Cu) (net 25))
 (segment (start 125.374998 119.220003) (end 125.374998 118.462182) (width 0.25) (layer F.Cu) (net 26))
 (segment (start 130.17218 113.665) (end 131.44218 113.665) (width 0.25) (layer F.Cu) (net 26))
 (segment (start 125.374998 118.462182) (end 130.17218 113.665) (width 0.25) (layer F.Cu) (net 26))
 (segment (start 133.35 111.75718) (end 133.35 110.49) (width 0.25) (layer F.Cu) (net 26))
 (segment (start 131.44218 113.665) (end 133.35 111.75718) (width 0.25) (layer F.Cu) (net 26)))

